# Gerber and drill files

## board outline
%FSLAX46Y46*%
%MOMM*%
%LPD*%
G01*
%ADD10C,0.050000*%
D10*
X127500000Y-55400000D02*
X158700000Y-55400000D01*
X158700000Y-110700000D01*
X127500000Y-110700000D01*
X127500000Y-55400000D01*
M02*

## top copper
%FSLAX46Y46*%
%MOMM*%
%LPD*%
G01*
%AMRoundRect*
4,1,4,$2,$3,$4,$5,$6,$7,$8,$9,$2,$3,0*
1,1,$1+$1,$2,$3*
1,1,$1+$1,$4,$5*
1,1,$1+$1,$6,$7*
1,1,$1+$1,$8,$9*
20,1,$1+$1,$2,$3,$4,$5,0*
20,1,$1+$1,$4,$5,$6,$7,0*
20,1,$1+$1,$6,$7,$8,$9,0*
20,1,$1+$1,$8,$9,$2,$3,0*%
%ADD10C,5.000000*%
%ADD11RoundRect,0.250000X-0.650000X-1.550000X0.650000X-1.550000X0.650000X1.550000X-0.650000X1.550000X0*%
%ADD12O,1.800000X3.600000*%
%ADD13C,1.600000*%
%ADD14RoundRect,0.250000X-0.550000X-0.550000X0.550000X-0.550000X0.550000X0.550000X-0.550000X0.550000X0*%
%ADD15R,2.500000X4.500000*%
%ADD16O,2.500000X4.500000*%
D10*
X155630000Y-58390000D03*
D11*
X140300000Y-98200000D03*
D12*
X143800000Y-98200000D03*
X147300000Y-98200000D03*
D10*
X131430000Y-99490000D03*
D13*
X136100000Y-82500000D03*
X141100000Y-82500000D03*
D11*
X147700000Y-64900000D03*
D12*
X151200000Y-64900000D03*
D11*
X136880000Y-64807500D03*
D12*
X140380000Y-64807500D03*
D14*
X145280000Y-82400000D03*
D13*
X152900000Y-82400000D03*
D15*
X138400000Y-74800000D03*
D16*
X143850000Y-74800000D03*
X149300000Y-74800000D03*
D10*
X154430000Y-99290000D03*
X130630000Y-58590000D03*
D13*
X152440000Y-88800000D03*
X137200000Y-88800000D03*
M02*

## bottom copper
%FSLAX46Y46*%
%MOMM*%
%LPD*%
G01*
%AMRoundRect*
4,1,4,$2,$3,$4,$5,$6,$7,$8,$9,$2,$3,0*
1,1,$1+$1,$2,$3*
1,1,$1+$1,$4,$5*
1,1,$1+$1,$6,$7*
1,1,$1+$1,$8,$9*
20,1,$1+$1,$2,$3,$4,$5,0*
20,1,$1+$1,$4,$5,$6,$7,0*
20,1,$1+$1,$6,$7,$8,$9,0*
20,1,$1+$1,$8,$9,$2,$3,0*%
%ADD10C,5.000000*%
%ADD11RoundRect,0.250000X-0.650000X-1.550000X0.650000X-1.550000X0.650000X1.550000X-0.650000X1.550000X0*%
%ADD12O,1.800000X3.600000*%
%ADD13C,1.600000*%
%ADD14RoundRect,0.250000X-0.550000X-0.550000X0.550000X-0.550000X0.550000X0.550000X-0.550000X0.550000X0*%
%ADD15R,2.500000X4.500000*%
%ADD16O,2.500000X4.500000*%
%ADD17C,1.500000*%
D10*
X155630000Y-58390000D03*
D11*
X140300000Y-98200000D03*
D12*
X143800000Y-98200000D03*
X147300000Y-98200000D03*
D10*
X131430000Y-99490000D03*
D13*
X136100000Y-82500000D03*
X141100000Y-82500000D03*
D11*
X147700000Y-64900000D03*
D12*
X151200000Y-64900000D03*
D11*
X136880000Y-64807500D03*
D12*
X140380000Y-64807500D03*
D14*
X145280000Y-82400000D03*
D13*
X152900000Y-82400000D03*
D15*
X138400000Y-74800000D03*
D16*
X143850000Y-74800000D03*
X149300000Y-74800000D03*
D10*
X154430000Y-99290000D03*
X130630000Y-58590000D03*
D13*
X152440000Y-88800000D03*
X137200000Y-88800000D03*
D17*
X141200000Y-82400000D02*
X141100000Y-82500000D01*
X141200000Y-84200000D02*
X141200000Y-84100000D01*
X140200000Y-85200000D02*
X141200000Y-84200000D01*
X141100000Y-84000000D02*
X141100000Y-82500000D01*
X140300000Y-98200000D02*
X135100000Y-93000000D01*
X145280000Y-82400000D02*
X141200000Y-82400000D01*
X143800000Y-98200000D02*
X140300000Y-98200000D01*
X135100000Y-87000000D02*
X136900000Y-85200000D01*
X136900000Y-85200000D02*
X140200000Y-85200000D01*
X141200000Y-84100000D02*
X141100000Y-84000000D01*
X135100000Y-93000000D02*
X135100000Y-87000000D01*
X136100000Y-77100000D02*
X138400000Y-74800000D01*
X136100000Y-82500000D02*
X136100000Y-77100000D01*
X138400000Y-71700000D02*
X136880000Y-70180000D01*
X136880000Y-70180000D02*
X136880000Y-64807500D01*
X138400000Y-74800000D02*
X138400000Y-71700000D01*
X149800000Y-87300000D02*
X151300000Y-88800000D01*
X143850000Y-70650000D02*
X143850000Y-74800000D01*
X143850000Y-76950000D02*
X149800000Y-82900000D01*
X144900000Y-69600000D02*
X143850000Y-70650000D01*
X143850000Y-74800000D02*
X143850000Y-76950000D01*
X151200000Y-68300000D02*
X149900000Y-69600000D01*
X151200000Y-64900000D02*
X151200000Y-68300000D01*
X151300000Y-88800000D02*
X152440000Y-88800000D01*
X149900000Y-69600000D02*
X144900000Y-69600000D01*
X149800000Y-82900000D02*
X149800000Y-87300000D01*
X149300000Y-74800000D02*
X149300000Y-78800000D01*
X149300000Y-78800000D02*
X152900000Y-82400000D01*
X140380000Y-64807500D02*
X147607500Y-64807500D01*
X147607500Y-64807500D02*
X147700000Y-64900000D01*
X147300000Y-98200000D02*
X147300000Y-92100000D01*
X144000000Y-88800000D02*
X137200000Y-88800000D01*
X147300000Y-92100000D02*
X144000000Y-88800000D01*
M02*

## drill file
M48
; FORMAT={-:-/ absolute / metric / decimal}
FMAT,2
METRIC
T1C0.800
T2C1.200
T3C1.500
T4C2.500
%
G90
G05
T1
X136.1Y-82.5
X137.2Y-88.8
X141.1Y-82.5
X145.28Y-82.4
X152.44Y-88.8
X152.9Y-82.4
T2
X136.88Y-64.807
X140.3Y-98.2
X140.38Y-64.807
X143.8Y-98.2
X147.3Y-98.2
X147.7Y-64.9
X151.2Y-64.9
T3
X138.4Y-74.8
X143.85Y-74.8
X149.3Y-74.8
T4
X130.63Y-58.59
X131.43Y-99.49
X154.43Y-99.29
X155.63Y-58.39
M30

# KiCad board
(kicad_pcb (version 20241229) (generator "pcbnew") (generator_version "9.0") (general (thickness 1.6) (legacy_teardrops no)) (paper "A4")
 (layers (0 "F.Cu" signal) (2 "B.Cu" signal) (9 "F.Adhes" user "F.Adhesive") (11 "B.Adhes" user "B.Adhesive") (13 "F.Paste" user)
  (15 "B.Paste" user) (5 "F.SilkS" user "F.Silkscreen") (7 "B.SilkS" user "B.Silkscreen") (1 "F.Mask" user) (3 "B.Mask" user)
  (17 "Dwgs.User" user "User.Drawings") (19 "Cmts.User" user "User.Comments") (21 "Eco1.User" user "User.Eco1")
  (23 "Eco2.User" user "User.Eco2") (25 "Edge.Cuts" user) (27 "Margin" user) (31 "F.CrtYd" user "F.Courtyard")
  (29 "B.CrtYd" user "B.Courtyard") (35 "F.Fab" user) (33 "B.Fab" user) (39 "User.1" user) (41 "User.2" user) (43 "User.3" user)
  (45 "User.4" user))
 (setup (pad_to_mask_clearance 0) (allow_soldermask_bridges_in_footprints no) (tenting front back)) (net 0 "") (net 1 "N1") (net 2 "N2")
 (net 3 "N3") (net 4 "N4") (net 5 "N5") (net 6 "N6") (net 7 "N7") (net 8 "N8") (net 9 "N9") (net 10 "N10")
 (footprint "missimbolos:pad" (layer "F.Cu") (at 155.6 58.4)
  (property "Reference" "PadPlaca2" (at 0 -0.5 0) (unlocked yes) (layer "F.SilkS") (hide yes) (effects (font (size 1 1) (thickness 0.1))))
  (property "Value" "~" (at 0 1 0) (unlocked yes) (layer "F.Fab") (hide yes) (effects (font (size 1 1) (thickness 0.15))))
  (pad "1" thru_hole circle (at 0.03 -0.01) (size 5 5) (drill 2.5) (layers "*.Cu" "*.Mask") (remove_unused_layers no) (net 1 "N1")))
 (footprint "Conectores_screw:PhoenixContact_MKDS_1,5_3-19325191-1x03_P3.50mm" (layer "F.Cu") (at 140.3 95.66)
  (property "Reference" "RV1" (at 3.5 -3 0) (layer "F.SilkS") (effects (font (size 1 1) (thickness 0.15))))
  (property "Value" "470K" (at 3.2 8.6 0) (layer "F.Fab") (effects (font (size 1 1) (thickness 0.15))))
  (pad "1" thru_hole roundrect (at 0 2.54) (size 1.8 3.6) (drill 1.2) (layers "*.Cu" "*.Mask") (remove_unused_layers no)
   (roundrect_rratio 0.138889) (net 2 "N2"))
  (pad "2" thru_hole oval (at 3.5 2.54) (size 1.8 3.6) (drill 1.2) (layers "*.Cu" "*.Mask") (remove_unused_layers no) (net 2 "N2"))
  (pad "3" thru_hole oval (at 7 2.54) (size 1.8 3.6) (drill 1.2) (layers "*.Cu" "*.Mask") (remove_unused_layers no) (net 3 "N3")))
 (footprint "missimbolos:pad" (layer "F.Cu") (at 131.4 99.5)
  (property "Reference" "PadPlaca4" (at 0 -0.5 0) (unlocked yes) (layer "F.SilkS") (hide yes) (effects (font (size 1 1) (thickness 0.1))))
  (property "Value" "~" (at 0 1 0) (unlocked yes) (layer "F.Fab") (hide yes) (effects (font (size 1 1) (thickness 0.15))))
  (pad "1" thru_hole circle (at 0.03 -0.01) (size 5 5) (drill 2.5) (layers "*.Cu" "*.Mask") (remove_unused_layers no) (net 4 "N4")))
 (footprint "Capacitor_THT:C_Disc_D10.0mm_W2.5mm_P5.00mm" (layer "F.Cu") (at 136.1 82.5)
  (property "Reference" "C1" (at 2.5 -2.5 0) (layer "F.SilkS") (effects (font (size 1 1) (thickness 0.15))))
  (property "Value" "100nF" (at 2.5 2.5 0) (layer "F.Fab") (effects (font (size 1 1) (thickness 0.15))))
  (pad "1" thru_hole circle (at 0 0) (size 1.6 1.6) (drill 0.8) (layers "*.Cu" "*.Mask") (remove_unused_layers no) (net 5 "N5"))
  (pad "2" thru_hole circle (at 5 0) (size 1.6 1.6) (drill 0.8) (layers "*.Cu" "*.Mask") (remove_unused_layers no) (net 2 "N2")))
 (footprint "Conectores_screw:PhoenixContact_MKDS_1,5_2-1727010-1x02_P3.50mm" (layer "F.Cu") (at 147.7 62.36)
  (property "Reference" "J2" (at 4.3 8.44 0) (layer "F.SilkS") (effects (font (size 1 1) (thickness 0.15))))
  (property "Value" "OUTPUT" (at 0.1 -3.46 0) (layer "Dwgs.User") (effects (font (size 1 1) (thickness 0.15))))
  (pad "1" thru_hole roundrect (at 0 2.54) (size 1.8 3.6) (drill 1.2) (layers "*.Cu" "*.Mask") (remove_unused_layers no)
   (roundrect_rratio 0.138889) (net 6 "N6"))
  (pad "2" thru_hole oval (at 3.5 2.54) (size 1.8 3.6) (drill 1.2) (layers "*.Cu" "*.Mask") (remove_unused_layers no) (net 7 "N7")))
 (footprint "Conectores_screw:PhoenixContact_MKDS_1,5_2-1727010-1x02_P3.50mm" (layer "F.Cu") (at 136.88 62.2675)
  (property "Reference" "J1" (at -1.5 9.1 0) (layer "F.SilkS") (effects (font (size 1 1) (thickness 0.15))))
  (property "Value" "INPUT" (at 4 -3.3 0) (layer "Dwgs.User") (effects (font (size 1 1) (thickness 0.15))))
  (pad "1" thru_hole roundrect (at 0 2.54) (size 1.8 3.6) (drill 1.2) (layers "*.Cu" "*.Mask") (remove_unused_layers no)
   (roundrect_rratio 0.138889) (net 5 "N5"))
  (pad "2" thru_hole oval (at 3.5 2.54) (size 1.8 3.6) (drill 1.2) (layers "*.Cu" "*.Mask") (remove_unused_layers no) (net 6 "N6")))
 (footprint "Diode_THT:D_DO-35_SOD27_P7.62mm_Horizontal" (layer "F.Cu") (at 145.28 82.4)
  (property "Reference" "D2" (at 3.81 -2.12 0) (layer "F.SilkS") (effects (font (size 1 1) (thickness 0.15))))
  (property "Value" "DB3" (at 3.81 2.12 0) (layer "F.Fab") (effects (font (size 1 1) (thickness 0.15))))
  (pad "1" thru_hole roundrect (at 0 0) (size 1.6 1.6) (drill 0.8) (layers "*.Cu" "*.Mask") (remove_unused_layers no)
   (roundrect_rratio 0.15625) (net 2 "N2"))
  (pad "2" thru_hole circle (at 7.62 0) (size 1.6 1.6) (drill 0.8) (layers "*.Cu" "*.Mask") (remove_unused_layers no) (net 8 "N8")))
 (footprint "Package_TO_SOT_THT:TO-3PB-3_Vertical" (layer "F.Cu") (at 138.4 74.8)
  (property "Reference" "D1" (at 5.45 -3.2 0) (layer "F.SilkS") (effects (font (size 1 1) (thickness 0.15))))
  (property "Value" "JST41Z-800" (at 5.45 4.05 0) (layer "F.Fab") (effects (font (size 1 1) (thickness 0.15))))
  (pad "1" thru_hole rect (at 0 0) (size 2.5 4.5) (drill 1.5) (layers "*.Cu" "*.Mask") (remove_unused_layers no) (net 5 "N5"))
  (pad "2" thru_hole oval (at 5.45 0) (size 2.5 4.5) (drill 1.5) (layers "*.Cu" "*.Mask") (remove_unused_layers no) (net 7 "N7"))
  (pad "3" thru_hole oval (at 10.9 0) (size 2.5 4.5) (drill 1.5) (layers "*.Cu" "*.Mask") (remove_unused_layers no) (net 8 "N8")))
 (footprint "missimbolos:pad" (layer "F.Cu") (at 154.4 99.3)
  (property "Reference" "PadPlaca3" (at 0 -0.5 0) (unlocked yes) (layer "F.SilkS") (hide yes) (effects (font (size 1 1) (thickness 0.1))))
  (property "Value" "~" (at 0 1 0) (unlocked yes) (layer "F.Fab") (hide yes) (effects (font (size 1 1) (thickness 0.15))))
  (pad "1" thru_hole circle (at 0.03 -0.01) (size 5 5) (drill 2.5) (layers "*.Cu" "*.Mask") (remove_unused_layers no) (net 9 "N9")))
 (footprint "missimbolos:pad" (layer "F.Cu") (at 130.6 58.6)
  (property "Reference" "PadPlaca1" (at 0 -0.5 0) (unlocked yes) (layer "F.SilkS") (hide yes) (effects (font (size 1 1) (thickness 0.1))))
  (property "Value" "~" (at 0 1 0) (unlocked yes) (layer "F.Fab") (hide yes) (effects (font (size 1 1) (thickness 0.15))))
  (pad "1" thru_hole circle (at 0.03 -0.01) (size 5 5) (drill 2.5) (layers "*.Cu" "*.Mask") (remove_unused_layers no) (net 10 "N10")))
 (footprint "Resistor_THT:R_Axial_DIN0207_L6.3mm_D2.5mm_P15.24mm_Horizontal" (layer "F.Cu") (at 152.44 88.8 180)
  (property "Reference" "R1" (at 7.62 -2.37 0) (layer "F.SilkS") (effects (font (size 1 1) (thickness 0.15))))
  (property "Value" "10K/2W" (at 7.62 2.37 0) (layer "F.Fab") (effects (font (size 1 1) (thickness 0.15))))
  (pad "1" thru_hole circle (at 0 0 180) (size 1.6 1.6) (drill 0.8) (layers "*.Cu" "*.Mask") (remove_unused_layers no) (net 7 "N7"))
  (pad "2" thru_hole circle (at 15.24 0 180) (size 1.6 1.6) (drill 0.8) (layers "*.Cu" "*.Mask") (remove_unused_layers no) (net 3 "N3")))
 (gr_rect (start 127.5 55.4) (end 158.7 110.7) (stroke (width 0.05) (type default)) (fill no) (layer "Edge.Cuts"))
 (segment (start 141.2 82.4) (end 141.1 82.5) (width 1.5) (layer "B.Cu") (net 2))
 (segment (start 141.2 84.2) (end 141.2 84.1) (width 1.5) (layer "B.Cu") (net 2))
 (segment (start 140.2 85.2) (end 141.2 84.2) (width 1.5) (layer "B.Cu") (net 2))
 (segment (start 141.1 84) (end 141.1 82.5) (width 1.5) (layer "B.Cu") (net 2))
 (segment (start 140.3 98.2) (end 135.1 93) (width 1.5) (layer "B.Cu") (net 2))
 (segment (start 145.28 82.4) (end 141.2 82.4) (width 1.5) (layer "B.Cu") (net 2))
 (segment (start 143.8 98.2) (end 140.3 98.2) (width 1.5) (layer "B.Cu") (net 2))
 (segment (start 135.1 87) (end 136.9 85.2) (width 1.5) (layer "B.Cu") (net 2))
 (segment (start 136.9 85.2) (end 140.2 85.2) (width 1.5) (layer "B.Cu") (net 2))
 (segment (start 141.2 84.1) (end 141.1 84) (width 1.5) (layer "B.Cu") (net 2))
 (segment (start 135.1 93) (end 135.1 87) (width 1.5) (layer "B.Cu") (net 2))
 (segment (start 136.1 77.1) (end 138.4 74.8) (width 1.5) (layer "B.Cu") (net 5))
 (segment (start 136.1 82.5) (end 136.1 77.1) (width 1.5) (layer "B.Cu") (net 5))
 (segment (start 138.4 71.7) (end 136.88 70.18) (width 1.5) (layer "B.Cu") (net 5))
 (segment (start 136.88 70.18) (end 136.88 64.8075) (width 1.5) (layer "B.Cu") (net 5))
 (segment (start 138.4 74.8) (end 138.4 71.7) (width 1.5) (layer "B.Cu") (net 5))
 (segment (start 149.8 87.3) (end 151.3 88.8) (width 1.5) (layer "B.Cu") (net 7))
 (segment (start 143.85 70.65) (end 143.85 74.8) (width 1.5) (layer "B.Cu") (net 7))
 (segment (start 143.85 76.95) (end 149.8 82.9) (width 1.5) (layer "B.Cu") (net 7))
 (segment (start 144.9 69.6) (end 143.85 70.65) (width 1.5) (layer "B.Cu") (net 7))
 (segment (start 143.85 74.8) (end 143.85 76.95) (width 1.5) (layer "B.Cu") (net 7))
 (segment (start 151.2 68.3) (end 149.9 69.6) (width 1.5) (layer "B.Cu") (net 7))
 (segment (start 151.2 64.9) (end 151.2 68.3) (width 1.5) (layer "B.Cu") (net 7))
 (segment (start 151.3 88.8) (end 152.44 88.8) (width 1.5) (layer "B.Cu") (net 7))
 (segment (start 149.9 69.6) (end 144.9 69.6) (width 1.5) (layer "B.Cu") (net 7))
 (segment (start 149.8 82.9) (end 149.8 87.3) (width 1.5) (layer "B.Cu") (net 7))
 (segment (start 149.3 74.8) (end 149.3 78.8) (width 1.5) (layer "B.Cu") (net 8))
 (segment (start 149.3 78.8) (end 152.9 82.4) (width 1.5) (layer "B.Cu") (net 8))
 (segment (start 140.38 64.8075) (end 147.6075 64.8075) (width 1.5) (layer "B.Cu") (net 6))
 (segment (start 147.6075 64.8075) (end 147.7 64.9) (width 1.5) (layer "B.Cu") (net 6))
 (segment (start 147.3 98.2) (end 147.3 92.1) (width 1.5) (layer "B.Cu") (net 3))
 (segment (start 144 88.8) (end 137.2 88.8) (width 1.5) (layer "B.Cu") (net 3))
 (segment (start 147.3 92.1) (end 144 88.8) (width 1.5) (layer "B.Cu") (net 3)))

